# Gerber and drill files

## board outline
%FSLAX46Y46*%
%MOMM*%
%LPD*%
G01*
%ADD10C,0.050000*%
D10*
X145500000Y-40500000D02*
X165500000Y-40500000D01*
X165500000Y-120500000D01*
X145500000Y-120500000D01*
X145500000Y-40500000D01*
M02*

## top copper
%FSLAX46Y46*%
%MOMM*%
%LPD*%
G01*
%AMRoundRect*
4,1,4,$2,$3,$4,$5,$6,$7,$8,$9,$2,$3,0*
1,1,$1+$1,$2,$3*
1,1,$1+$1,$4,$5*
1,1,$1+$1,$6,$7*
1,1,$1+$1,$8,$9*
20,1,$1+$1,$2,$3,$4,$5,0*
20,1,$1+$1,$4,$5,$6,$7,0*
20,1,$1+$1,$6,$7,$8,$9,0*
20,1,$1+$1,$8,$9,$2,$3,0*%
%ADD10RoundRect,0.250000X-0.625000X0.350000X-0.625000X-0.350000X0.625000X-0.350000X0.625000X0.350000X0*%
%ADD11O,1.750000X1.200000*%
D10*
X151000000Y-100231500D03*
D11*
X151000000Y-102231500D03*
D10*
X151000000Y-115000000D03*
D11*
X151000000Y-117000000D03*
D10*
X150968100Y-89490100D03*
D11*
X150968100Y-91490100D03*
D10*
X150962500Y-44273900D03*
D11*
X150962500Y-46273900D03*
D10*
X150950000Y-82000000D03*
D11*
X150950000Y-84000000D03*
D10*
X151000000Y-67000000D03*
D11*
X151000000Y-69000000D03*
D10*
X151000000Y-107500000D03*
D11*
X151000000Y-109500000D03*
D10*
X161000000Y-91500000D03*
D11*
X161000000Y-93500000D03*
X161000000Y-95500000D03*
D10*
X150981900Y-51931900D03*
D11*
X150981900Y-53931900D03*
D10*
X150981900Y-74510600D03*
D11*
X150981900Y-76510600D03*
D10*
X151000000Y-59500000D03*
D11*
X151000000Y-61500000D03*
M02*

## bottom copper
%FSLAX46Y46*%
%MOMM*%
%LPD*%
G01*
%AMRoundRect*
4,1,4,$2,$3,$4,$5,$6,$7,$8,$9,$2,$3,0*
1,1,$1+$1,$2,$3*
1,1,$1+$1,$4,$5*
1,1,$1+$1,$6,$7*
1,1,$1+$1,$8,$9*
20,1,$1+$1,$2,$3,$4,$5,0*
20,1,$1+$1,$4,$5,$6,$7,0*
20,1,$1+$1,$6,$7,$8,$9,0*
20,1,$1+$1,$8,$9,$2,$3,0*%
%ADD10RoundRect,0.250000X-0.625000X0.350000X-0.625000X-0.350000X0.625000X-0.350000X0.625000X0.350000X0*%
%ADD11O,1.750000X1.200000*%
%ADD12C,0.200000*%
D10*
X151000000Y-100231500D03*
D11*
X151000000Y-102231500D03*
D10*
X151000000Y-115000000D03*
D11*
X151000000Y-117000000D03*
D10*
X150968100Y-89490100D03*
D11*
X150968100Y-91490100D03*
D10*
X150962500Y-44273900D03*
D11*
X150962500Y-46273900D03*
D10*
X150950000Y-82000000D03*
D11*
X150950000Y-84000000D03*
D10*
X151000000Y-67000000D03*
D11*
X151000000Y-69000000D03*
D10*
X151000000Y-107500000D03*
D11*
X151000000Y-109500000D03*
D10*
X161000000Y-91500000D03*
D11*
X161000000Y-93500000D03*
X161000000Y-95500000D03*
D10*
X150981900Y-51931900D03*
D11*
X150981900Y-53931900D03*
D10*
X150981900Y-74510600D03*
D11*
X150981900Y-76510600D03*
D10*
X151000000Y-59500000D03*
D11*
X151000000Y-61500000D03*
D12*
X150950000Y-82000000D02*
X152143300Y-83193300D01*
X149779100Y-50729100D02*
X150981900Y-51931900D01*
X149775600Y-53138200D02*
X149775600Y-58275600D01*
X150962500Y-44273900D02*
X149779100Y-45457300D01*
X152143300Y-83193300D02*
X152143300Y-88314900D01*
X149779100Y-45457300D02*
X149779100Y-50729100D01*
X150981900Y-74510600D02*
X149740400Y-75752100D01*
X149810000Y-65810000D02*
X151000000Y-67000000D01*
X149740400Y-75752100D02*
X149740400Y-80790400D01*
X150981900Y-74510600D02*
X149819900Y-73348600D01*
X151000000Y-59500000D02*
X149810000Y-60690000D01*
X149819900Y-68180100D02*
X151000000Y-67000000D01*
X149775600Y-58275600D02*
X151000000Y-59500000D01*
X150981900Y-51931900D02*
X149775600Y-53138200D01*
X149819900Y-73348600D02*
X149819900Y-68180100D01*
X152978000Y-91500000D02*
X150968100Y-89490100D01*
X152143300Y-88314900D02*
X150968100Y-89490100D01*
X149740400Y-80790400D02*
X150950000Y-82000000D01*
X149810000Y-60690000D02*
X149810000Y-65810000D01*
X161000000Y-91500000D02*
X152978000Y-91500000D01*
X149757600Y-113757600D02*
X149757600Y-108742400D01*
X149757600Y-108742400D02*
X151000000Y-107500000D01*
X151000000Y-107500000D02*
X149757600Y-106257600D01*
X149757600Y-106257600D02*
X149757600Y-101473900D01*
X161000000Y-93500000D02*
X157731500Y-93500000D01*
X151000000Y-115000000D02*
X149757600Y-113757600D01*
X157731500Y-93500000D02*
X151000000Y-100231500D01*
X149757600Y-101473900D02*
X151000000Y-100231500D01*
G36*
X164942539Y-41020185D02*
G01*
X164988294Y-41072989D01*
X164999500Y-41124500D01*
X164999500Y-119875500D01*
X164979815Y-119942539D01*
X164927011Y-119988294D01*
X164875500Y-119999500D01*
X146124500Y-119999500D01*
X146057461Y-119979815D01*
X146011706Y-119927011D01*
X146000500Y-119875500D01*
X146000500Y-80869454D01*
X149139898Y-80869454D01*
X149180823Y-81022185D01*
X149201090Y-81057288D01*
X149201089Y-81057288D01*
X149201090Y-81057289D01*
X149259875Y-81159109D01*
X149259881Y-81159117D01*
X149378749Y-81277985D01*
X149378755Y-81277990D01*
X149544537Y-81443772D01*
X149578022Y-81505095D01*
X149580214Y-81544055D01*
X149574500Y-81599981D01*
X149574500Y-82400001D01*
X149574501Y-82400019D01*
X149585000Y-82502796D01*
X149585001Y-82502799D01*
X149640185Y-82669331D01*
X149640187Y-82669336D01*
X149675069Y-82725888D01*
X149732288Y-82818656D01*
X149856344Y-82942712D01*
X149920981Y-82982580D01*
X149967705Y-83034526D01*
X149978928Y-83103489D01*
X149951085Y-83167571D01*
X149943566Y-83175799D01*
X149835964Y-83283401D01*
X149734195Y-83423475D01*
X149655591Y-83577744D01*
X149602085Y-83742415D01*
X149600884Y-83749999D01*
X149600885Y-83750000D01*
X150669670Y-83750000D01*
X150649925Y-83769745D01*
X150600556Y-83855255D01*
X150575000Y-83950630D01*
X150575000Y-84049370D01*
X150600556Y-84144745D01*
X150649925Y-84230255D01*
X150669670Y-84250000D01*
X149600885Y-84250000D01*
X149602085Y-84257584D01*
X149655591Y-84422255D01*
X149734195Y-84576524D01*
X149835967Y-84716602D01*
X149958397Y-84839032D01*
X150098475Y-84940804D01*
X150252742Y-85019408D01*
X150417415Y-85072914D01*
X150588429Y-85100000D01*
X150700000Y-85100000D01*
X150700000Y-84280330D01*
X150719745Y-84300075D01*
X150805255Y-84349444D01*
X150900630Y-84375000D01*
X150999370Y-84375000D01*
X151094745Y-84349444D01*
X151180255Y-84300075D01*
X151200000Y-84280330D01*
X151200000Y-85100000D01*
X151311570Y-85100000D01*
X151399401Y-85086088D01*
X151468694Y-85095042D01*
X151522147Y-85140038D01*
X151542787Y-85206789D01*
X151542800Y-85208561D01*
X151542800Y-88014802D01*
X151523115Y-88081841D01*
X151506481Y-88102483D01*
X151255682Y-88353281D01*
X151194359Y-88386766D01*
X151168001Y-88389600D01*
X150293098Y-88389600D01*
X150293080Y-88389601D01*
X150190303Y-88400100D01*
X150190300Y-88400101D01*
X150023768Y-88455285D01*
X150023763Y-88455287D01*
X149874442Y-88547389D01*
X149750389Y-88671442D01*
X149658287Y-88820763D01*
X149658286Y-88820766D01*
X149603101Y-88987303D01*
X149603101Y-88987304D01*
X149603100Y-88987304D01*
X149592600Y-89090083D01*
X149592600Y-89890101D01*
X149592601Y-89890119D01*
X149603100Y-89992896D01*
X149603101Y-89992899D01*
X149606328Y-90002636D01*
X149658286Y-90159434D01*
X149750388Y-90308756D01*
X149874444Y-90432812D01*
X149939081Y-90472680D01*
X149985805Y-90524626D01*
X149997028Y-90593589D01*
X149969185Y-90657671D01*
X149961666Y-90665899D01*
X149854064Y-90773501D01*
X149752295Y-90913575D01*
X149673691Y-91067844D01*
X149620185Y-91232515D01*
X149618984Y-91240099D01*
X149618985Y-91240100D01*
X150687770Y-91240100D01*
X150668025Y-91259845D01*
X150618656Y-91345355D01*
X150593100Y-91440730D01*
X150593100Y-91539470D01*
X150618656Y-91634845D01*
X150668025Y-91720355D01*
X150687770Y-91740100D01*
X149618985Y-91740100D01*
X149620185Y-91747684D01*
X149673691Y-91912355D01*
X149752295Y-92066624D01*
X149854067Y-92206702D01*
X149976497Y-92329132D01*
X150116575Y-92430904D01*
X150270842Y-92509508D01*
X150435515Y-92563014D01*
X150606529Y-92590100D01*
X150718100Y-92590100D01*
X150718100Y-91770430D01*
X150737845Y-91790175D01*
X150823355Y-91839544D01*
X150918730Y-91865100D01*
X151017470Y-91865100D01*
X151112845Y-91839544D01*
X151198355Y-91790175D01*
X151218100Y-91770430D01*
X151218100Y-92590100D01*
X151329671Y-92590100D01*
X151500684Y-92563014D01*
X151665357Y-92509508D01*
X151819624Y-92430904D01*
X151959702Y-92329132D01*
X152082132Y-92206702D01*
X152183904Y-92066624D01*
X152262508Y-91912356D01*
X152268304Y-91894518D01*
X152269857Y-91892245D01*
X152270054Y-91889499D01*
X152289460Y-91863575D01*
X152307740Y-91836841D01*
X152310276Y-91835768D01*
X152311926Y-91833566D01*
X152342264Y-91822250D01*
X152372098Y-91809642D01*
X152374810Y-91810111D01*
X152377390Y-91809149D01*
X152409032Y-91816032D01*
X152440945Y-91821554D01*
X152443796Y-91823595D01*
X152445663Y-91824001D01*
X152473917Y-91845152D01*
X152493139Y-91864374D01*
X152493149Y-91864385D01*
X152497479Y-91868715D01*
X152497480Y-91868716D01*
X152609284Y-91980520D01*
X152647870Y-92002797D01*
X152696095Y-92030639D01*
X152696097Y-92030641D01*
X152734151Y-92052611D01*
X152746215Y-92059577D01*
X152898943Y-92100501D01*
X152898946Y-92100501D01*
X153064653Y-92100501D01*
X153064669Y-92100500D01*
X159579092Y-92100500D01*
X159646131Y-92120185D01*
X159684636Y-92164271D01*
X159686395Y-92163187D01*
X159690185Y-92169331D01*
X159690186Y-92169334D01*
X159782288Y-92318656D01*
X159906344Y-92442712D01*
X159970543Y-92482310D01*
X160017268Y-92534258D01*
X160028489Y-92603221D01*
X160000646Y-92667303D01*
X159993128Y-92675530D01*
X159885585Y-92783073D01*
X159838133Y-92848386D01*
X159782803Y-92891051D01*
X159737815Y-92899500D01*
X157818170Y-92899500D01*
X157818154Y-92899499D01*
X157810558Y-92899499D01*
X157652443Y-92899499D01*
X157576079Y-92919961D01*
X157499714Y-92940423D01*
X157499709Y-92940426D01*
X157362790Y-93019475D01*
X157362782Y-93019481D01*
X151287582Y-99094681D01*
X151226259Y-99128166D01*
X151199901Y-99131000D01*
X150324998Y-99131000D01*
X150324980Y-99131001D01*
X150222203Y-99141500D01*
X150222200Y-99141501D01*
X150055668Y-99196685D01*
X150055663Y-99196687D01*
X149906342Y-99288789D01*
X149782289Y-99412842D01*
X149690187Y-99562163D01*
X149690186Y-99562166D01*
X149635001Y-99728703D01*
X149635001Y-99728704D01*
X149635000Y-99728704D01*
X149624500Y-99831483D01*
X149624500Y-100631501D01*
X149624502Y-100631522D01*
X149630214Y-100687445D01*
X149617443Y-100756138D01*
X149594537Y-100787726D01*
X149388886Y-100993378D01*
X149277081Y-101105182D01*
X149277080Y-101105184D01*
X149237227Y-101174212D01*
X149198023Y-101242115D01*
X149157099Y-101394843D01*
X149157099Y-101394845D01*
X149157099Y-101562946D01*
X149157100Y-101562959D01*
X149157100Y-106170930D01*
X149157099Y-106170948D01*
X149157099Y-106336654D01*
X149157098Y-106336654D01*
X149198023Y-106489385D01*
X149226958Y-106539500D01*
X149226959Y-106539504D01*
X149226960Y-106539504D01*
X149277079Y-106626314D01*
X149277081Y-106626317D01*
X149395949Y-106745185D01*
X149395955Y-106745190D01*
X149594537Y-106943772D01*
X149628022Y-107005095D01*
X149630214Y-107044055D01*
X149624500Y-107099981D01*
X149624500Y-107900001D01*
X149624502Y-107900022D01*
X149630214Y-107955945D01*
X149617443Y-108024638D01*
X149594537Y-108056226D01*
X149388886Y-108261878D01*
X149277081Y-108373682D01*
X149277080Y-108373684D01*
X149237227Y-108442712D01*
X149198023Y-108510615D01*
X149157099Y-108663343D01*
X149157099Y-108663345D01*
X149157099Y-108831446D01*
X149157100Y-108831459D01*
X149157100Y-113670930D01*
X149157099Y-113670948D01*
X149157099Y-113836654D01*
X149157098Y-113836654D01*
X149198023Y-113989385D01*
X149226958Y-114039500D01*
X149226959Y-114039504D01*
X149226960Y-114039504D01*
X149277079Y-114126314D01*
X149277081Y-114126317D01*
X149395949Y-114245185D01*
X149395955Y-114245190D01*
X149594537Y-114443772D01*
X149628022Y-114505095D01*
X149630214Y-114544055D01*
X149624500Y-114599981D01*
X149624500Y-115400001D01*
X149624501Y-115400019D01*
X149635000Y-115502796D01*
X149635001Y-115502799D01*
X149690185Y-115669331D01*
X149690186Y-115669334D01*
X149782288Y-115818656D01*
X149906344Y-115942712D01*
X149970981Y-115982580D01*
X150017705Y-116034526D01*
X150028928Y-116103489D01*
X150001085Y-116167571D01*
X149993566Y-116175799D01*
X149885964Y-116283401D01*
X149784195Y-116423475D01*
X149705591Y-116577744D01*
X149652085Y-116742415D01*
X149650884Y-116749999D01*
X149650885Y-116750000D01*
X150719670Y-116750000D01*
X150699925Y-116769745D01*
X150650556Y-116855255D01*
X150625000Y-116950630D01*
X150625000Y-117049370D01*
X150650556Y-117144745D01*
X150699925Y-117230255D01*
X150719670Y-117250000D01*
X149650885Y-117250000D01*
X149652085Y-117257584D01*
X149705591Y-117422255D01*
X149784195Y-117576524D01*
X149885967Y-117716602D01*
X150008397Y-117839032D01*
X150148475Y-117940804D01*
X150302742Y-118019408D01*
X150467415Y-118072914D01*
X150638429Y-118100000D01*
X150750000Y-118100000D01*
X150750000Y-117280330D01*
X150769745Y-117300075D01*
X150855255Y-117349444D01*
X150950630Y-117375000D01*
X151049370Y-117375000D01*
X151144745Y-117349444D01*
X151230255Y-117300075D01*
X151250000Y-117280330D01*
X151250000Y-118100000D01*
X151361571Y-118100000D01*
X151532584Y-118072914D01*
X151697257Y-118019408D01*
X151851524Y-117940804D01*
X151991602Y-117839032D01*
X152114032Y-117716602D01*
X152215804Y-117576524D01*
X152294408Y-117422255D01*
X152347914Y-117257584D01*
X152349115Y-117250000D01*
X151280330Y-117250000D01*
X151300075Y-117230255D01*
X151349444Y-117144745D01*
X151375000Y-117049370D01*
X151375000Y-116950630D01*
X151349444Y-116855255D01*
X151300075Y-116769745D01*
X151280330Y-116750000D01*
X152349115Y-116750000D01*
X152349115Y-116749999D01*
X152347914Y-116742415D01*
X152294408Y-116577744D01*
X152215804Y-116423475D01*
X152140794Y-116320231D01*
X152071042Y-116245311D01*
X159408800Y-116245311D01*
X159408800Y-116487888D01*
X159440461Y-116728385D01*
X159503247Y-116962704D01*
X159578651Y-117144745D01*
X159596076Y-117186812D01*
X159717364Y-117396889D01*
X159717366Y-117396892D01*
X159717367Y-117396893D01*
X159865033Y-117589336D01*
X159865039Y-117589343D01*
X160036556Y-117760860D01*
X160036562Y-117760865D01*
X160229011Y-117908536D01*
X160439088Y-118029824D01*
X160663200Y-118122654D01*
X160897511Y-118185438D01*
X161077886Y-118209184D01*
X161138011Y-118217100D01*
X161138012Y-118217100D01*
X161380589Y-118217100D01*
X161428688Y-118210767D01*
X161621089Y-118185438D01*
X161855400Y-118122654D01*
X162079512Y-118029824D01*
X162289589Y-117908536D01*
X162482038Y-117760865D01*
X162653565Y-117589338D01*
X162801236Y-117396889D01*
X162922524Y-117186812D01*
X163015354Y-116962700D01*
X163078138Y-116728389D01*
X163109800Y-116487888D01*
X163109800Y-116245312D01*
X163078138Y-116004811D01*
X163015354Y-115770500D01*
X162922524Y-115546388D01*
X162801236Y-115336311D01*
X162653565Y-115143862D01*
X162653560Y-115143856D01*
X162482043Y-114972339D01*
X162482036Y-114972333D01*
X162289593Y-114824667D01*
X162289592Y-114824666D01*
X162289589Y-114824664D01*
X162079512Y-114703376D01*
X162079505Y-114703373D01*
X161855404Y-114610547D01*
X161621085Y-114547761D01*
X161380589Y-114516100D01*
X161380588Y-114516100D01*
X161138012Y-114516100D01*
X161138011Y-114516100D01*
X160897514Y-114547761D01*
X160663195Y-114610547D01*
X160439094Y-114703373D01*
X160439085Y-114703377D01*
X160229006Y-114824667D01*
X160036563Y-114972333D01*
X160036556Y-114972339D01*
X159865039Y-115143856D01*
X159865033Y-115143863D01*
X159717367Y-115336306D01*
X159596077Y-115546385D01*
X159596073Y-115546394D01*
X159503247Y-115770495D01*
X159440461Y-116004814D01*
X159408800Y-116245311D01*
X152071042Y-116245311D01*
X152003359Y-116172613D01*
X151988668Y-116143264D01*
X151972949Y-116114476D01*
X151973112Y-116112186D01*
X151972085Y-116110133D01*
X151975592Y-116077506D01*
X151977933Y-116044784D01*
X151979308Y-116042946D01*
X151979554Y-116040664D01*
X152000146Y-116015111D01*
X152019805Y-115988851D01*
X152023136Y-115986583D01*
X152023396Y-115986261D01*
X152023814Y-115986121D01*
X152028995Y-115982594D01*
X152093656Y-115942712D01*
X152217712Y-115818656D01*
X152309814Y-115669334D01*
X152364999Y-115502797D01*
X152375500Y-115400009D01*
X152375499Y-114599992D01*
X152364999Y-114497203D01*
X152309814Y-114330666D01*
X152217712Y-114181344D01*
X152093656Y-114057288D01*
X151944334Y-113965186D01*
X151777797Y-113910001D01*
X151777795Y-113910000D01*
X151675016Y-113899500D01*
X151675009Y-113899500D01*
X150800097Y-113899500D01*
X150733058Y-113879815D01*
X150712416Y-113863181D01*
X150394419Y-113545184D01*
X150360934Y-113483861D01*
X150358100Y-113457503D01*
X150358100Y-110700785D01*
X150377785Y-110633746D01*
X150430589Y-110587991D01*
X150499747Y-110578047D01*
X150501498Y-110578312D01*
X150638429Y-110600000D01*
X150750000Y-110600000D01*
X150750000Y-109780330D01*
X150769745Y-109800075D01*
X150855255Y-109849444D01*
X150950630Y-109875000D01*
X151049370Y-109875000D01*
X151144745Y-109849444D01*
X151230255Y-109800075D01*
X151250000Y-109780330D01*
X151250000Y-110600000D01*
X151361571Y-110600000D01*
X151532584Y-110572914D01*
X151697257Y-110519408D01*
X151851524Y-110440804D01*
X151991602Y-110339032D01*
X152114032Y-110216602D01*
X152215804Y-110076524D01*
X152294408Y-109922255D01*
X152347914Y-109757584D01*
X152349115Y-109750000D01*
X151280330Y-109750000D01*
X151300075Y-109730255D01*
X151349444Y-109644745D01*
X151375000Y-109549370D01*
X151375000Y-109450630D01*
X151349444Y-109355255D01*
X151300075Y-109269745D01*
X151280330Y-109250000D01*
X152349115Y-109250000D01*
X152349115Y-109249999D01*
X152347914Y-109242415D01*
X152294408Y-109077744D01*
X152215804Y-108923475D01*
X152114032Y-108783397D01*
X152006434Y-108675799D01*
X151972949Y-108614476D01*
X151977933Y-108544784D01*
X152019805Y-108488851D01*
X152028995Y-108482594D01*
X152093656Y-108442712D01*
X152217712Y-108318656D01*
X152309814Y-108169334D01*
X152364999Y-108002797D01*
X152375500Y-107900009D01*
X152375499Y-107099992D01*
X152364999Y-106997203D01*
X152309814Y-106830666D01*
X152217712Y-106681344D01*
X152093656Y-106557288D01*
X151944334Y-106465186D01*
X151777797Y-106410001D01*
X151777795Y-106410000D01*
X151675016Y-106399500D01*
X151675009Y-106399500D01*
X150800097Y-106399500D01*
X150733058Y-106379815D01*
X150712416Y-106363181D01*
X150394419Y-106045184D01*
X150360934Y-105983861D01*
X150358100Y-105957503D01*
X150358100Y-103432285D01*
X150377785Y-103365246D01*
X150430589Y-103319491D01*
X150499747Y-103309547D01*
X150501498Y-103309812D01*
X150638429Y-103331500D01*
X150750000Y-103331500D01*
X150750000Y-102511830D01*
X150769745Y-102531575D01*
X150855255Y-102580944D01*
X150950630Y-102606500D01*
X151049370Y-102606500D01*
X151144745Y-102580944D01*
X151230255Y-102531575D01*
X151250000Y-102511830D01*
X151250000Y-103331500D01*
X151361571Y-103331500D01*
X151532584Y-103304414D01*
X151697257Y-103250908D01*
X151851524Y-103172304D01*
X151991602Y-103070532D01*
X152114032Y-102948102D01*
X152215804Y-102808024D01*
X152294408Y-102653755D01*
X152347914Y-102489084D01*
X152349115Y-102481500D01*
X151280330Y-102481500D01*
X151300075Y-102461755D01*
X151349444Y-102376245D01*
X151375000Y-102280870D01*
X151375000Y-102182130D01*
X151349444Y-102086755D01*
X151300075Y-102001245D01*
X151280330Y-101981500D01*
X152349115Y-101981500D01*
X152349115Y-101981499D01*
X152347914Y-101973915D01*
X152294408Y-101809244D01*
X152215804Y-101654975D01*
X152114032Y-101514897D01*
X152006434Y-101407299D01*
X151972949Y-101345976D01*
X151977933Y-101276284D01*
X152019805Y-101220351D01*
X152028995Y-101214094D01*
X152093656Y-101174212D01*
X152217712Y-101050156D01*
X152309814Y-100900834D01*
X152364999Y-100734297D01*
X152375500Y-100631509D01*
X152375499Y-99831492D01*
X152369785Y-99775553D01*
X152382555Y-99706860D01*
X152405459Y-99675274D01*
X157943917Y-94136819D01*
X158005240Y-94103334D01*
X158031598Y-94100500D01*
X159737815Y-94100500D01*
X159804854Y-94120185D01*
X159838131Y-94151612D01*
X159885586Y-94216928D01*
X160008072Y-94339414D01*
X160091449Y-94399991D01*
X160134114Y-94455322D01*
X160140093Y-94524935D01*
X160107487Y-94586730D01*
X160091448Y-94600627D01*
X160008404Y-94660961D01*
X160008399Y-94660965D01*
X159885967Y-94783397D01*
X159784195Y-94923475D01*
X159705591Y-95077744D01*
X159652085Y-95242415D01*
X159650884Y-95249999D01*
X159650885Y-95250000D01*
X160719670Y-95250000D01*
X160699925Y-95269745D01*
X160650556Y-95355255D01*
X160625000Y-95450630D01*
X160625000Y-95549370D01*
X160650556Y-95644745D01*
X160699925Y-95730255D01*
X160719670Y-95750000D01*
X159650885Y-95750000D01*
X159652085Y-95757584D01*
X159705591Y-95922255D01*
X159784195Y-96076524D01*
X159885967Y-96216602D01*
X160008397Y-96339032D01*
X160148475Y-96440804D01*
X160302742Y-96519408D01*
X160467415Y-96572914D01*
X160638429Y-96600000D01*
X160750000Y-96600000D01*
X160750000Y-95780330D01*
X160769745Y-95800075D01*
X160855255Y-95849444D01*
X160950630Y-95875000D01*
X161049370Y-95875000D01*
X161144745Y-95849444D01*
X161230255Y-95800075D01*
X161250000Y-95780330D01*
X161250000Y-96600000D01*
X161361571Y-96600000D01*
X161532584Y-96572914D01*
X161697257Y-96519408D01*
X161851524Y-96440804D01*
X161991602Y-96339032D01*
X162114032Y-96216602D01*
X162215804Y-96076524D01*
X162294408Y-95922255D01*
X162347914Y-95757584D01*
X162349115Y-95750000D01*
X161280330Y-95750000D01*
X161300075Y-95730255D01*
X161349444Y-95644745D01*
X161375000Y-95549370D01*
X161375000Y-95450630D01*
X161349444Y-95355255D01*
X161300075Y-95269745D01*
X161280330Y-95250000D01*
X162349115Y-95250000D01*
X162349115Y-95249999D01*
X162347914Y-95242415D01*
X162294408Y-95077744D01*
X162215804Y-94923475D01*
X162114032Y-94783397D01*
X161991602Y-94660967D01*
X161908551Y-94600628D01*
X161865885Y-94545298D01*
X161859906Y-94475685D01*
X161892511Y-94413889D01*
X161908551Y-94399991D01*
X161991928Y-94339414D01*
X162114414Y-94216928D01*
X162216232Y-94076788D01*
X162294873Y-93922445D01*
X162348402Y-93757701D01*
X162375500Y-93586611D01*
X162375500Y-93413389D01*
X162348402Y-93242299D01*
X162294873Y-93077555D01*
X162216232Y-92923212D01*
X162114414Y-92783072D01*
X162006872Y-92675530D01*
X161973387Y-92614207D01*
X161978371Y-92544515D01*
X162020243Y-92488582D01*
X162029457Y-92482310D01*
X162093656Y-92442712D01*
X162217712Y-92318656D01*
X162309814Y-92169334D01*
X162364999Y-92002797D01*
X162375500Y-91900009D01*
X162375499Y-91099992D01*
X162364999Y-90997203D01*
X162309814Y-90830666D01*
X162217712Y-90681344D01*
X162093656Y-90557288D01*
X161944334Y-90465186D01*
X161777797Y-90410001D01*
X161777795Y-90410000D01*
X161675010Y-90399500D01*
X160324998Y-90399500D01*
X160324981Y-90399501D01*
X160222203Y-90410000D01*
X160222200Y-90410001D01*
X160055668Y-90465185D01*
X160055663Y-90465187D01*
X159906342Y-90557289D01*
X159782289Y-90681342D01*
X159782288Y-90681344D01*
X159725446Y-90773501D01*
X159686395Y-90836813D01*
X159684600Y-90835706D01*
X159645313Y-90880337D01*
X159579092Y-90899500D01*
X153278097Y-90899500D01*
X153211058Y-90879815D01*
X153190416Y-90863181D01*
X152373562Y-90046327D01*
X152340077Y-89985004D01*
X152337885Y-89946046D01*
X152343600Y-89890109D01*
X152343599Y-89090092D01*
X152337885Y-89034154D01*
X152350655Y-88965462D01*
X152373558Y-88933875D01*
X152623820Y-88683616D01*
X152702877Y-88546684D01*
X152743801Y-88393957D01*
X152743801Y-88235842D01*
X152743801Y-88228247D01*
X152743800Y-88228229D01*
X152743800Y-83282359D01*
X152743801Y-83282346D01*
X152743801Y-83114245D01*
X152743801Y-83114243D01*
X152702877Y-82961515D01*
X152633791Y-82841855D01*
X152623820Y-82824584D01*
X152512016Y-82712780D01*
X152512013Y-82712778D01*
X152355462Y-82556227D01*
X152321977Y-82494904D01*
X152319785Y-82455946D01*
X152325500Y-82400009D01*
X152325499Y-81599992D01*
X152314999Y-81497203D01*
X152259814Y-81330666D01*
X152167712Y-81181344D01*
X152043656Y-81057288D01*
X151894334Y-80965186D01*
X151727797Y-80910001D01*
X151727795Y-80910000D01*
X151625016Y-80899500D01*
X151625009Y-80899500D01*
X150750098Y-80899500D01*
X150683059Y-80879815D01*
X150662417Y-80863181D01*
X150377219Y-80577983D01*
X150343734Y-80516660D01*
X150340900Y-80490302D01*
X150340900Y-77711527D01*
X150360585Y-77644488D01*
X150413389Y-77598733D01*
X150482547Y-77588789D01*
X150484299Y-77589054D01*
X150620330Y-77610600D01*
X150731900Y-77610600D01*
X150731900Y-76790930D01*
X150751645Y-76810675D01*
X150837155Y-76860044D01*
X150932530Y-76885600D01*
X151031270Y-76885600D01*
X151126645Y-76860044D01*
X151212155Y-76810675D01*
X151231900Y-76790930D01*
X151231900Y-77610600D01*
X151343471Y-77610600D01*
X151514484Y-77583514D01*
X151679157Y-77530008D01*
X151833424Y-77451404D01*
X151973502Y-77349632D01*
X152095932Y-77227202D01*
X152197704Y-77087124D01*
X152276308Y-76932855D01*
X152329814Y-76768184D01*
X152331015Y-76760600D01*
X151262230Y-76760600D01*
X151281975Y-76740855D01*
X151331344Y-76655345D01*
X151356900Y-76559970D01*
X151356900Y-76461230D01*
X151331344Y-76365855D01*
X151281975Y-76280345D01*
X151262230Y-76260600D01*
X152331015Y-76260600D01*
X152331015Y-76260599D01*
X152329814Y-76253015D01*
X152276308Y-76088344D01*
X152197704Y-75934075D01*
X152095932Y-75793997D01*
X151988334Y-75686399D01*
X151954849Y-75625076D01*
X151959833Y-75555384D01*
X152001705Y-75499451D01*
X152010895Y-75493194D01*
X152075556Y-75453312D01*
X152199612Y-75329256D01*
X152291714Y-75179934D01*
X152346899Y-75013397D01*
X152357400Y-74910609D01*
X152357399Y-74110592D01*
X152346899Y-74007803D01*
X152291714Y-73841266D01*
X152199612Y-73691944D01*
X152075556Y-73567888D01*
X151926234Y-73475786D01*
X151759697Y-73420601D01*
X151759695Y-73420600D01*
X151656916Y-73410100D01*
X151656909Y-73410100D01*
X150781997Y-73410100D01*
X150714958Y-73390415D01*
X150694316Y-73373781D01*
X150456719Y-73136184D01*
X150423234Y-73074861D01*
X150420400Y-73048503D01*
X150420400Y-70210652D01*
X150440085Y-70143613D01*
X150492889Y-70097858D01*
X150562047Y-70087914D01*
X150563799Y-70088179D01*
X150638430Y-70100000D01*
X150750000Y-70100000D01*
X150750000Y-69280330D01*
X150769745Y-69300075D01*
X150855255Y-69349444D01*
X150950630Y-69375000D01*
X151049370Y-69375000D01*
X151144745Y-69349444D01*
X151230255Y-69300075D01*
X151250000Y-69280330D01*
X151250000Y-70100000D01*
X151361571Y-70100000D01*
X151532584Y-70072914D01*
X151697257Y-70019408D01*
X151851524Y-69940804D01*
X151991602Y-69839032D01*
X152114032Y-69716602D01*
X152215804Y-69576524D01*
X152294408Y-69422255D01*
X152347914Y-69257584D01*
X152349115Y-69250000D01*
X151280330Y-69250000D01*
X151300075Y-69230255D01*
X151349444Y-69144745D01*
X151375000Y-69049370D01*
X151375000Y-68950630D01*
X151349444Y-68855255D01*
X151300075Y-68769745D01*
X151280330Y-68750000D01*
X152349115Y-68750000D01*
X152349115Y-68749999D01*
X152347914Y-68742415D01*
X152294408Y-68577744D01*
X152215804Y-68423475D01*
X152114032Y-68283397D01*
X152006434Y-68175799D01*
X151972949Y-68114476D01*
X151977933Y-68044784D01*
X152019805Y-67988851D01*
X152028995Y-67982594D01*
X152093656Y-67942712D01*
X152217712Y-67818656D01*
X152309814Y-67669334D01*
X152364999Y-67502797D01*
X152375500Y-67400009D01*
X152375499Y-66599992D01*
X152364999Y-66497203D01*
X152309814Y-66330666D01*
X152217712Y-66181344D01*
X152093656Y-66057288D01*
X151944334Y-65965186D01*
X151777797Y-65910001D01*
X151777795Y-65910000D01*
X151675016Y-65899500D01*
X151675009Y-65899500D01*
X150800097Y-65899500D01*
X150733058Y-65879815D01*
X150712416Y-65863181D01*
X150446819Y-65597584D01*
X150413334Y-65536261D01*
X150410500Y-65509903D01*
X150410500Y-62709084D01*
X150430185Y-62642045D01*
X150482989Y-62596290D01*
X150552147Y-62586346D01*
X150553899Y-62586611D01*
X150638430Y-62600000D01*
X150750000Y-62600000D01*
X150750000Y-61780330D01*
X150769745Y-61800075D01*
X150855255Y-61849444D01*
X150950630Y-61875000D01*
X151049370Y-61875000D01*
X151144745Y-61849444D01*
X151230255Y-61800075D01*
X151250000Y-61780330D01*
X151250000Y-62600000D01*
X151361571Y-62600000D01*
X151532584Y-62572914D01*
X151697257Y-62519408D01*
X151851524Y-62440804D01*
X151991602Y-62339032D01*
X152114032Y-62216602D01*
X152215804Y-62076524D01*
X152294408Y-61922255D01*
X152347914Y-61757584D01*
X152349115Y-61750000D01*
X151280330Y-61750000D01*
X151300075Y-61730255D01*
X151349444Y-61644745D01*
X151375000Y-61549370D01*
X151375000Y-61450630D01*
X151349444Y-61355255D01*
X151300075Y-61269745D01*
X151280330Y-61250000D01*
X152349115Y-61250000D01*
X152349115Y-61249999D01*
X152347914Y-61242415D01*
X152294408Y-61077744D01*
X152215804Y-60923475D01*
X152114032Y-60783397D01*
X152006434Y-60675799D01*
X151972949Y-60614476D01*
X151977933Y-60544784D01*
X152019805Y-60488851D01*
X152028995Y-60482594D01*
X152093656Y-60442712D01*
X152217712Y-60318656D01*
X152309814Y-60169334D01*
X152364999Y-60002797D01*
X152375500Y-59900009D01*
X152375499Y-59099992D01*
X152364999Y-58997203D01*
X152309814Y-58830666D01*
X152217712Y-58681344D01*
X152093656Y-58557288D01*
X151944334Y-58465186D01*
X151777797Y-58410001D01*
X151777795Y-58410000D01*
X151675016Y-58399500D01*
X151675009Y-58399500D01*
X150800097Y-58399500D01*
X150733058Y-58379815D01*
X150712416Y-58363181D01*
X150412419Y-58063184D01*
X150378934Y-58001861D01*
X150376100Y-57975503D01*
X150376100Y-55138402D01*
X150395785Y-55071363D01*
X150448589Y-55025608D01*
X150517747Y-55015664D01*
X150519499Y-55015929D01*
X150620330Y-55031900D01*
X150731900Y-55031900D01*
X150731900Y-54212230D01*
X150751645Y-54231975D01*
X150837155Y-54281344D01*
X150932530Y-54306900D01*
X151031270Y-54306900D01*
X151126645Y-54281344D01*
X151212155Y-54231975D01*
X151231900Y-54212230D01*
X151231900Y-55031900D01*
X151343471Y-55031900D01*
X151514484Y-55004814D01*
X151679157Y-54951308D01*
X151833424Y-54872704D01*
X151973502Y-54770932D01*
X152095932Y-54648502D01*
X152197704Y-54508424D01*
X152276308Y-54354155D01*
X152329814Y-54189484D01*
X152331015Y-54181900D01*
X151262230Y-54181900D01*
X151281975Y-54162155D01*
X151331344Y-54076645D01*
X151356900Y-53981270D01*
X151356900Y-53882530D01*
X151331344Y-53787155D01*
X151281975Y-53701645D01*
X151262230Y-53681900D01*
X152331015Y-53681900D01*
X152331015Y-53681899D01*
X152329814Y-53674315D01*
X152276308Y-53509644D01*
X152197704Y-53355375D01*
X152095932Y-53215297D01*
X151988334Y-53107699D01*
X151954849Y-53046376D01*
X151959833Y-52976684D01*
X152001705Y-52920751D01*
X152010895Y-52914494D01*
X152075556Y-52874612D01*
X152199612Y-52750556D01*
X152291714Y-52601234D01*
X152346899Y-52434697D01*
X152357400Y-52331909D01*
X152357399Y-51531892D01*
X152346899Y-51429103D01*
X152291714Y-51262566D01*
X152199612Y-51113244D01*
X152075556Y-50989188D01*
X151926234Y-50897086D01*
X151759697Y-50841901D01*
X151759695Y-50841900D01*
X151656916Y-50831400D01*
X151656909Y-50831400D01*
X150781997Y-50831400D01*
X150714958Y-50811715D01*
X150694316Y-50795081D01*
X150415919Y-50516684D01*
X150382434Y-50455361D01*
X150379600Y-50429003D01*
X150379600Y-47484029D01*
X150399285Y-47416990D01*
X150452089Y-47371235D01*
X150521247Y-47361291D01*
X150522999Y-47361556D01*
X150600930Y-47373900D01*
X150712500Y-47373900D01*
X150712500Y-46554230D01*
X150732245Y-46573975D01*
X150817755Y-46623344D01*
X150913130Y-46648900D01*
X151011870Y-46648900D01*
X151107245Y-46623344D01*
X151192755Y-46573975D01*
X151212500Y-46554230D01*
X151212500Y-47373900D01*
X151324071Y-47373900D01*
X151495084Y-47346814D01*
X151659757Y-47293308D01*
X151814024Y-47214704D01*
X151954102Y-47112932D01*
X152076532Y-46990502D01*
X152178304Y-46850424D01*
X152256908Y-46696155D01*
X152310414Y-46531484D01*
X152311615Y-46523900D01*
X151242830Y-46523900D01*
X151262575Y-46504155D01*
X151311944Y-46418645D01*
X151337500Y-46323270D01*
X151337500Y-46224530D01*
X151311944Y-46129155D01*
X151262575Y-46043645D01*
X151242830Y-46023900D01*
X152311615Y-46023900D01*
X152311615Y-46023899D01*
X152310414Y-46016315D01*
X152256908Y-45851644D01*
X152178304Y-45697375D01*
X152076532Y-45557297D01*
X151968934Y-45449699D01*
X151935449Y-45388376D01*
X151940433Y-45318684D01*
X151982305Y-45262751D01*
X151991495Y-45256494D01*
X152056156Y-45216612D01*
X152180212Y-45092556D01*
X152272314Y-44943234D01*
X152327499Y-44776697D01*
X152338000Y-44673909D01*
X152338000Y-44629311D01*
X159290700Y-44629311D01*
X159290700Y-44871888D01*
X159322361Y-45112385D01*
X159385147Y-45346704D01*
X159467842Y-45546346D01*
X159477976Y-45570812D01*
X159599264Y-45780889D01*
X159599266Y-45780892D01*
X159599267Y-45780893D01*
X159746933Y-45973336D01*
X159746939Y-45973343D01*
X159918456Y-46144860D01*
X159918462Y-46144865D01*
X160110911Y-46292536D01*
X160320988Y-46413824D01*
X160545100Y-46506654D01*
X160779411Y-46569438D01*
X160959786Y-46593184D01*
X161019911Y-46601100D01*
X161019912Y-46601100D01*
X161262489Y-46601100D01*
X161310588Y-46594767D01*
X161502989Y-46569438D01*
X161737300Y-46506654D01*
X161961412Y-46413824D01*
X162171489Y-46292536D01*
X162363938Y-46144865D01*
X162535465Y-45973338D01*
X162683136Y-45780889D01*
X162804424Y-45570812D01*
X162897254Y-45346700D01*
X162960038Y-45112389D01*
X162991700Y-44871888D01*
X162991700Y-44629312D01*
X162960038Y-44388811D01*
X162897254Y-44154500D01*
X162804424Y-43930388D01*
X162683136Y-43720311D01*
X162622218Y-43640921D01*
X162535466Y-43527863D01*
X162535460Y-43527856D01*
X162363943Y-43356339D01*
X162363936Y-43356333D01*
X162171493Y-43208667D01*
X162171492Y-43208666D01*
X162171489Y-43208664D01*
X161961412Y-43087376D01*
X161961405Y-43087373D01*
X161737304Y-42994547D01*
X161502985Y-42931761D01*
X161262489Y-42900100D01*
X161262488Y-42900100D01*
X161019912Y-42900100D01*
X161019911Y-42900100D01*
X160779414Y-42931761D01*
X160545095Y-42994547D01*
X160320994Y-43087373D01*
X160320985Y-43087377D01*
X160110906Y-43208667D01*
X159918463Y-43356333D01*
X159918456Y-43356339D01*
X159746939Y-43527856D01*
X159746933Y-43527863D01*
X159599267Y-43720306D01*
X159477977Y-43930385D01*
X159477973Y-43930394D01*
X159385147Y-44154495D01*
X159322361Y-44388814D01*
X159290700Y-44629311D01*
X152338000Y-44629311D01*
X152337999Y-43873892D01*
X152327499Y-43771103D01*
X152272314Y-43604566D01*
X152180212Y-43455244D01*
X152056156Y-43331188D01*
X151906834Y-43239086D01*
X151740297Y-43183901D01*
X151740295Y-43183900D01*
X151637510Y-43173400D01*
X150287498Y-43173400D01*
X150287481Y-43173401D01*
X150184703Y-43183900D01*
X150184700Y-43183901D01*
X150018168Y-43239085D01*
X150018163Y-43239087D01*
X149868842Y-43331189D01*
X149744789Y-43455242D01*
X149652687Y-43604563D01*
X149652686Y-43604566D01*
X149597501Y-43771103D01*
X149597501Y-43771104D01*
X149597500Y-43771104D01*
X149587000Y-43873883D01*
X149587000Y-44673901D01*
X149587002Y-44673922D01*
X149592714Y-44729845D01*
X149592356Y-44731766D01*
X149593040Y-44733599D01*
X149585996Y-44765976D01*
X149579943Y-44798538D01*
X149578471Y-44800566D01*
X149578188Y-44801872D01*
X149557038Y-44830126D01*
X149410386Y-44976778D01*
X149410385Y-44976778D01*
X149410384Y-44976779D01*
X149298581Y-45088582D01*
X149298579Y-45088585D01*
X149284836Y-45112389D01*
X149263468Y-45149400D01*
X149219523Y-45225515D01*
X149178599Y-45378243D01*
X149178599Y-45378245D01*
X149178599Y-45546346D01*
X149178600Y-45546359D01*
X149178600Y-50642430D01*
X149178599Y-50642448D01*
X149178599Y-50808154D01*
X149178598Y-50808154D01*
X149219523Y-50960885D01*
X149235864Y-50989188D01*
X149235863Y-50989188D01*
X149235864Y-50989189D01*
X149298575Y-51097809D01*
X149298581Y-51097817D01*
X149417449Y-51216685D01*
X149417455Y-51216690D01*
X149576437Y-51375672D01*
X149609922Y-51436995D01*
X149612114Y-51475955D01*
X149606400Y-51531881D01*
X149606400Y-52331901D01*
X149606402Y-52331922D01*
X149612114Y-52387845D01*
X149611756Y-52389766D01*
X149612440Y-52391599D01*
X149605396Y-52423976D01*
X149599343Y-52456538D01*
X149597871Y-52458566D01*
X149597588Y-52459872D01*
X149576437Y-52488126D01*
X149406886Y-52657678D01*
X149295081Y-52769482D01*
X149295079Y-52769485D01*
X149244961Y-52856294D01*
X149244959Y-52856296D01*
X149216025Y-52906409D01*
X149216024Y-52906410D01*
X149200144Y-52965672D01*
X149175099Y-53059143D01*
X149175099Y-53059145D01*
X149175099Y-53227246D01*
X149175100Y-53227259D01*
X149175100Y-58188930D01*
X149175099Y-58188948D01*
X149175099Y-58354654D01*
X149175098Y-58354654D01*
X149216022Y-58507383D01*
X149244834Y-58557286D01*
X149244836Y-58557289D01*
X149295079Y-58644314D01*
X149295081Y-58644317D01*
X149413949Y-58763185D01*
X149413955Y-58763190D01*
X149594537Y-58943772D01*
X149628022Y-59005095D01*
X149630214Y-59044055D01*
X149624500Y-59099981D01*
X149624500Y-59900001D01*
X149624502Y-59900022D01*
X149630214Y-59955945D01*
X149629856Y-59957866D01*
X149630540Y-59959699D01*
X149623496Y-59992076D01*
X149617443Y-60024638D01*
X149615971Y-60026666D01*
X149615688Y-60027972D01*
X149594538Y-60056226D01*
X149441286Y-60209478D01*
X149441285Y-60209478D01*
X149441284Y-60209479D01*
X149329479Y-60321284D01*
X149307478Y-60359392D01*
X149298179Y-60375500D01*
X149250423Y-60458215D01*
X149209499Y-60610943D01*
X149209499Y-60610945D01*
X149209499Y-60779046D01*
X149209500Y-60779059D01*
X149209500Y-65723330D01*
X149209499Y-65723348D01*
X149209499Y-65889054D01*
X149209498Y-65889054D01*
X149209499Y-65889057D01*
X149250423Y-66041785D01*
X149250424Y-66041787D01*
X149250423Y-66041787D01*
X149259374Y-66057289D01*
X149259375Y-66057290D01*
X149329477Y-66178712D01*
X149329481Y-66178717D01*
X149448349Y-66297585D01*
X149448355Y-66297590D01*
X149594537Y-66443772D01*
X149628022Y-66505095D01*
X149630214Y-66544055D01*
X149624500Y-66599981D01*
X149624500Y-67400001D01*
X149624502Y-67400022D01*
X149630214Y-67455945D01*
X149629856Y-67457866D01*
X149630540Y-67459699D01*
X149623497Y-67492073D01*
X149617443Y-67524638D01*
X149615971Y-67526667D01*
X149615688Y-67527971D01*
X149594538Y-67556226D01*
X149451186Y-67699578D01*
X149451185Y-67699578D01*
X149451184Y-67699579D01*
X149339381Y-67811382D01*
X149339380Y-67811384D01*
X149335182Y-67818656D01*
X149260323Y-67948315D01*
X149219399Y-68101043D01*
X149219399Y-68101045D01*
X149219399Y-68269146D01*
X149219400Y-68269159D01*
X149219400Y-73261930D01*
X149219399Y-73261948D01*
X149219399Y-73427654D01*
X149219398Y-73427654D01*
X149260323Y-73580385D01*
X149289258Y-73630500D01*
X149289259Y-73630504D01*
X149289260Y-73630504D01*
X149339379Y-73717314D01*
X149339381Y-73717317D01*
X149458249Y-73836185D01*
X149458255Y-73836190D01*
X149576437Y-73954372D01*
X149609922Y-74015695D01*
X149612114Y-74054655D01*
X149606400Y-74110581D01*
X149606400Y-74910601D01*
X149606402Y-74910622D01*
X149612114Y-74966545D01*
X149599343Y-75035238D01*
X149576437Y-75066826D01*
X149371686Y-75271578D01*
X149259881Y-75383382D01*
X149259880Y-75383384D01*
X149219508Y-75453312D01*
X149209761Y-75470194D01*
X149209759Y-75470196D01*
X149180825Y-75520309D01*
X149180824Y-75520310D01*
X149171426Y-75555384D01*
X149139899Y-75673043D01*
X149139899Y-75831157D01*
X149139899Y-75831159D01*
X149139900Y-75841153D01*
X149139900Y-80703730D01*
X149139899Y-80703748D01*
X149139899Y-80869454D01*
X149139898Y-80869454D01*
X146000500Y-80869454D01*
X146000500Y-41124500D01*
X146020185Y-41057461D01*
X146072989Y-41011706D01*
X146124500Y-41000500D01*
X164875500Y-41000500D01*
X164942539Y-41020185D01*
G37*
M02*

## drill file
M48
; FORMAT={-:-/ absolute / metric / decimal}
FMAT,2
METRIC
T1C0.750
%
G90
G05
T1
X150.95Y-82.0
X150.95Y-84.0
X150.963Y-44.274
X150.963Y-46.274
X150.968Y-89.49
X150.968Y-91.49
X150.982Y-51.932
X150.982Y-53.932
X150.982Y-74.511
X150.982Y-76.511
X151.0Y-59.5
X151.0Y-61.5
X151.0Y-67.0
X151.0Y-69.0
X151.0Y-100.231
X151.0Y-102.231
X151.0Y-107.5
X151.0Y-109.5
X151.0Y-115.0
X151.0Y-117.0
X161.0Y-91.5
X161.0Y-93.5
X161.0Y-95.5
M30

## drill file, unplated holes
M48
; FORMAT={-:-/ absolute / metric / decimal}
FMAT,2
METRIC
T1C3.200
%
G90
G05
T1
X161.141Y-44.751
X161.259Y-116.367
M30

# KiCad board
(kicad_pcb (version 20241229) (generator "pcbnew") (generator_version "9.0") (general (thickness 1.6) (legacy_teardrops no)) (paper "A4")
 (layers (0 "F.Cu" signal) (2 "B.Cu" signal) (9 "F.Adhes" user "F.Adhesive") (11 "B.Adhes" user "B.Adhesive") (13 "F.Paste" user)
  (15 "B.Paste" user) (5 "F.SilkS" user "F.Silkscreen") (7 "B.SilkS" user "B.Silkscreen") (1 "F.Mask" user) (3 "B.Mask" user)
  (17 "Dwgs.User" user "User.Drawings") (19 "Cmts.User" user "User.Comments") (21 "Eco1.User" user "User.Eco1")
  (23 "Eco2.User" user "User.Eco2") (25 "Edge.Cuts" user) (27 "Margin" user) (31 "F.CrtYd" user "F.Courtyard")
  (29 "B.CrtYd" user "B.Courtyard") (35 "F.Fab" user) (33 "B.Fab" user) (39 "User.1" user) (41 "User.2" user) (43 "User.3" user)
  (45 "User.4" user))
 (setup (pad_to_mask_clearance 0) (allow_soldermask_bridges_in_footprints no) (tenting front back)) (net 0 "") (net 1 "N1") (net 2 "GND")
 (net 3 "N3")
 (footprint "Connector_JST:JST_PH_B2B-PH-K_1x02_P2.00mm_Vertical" (layer "F.Cu") (at 151 100.2315 -90)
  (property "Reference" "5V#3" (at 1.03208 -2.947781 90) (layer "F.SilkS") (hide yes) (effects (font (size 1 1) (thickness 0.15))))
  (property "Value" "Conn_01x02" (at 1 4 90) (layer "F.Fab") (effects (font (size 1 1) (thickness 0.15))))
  (pad "1" thru_hole roundrect (at 0 0 270) (size 1.2 1.75) (drill 0.75) (layers "*.Cu" "*.Mask") (remove_unused_layers no)
   (roundrect_rratio 0.208333) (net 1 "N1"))
  (pad "2" thru_hole oval (at 2 0 270) (size 1.2 1.75) (drill 0.75) (layers "*.Cu" "*.Mask") (remove_unused_layers no) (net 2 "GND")))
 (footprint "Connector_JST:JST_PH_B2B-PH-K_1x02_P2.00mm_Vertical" (layer "F.Cu") (at 151 115 -90)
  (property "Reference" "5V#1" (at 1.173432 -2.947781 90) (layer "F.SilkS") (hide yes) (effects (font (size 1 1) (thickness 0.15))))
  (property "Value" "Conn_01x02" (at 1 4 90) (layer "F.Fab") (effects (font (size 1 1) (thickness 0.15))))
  (pad "1" thru_hole roundrect (at 0 0 270) (size 1.2 1.75) (drill 0.75) (layers "*.Cu" "*.Mask") (remove_unused_layers no)
   (roundrect_rratio 0.208333) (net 1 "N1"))
  (pad "2" thru_hole oval (at 2 0 270) (size 1.2 1.75) (drill 0.75) (layers "*.Cu" "*.Mask") (remove_unused_layers no) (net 2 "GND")))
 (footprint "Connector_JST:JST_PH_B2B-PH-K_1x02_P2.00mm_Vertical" (layer "F.Cu") (at 150.9681 89.4901 -90)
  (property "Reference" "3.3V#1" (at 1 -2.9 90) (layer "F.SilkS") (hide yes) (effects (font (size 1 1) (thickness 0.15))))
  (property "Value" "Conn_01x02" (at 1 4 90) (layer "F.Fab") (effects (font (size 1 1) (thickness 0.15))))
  (pad "1" thru_hole roundrect (at 0 0 270) (size 1.2 1.75) (drill 0.75) (layers "*.Cu" "*.Mask") (remove_unused_layers no)
   (roundrect_rratio 0.208333) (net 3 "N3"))
  (pad "2" thru_hole oval (at 2 0 270) (size 1.2 1.75) (drill 0.75) (layers "*.Cu" "*.Mask") (remove_unused_layers no) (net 2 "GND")))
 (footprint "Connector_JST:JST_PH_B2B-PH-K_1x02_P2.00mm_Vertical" (layer "F.Cu") (at 150.9625 44.2739 -90)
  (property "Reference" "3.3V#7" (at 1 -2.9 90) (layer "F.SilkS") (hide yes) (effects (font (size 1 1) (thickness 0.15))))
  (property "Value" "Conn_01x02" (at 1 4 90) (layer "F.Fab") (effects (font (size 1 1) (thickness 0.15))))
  (pad "1" thru_hole roundrect (at 0 0 270) (size 1.2 1.75) (drill 0.75) (layers "*.Cu" "*.Mask") (remove_unused_layers no)
   (roundrect_rratio 0.208333) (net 3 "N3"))
  (pad "2" thru_hole oval (at 2 0 270) (size 1.2 1.75) (drill 0.75) (layers "*.Cu" "*.Mask") (remove_unused_layers no) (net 2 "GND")))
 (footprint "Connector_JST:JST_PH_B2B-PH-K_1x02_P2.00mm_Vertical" (layer "F.Cu") (at 150.95 82 -90)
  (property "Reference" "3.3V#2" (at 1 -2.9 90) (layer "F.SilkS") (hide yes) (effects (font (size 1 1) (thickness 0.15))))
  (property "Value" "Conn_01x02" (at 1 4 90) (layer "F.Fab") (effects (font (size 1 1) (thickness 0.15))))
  (pad "1" thru_hole roundrect (at 0 0 270) (size 1.2 1.75) (drill 0.75) (layers "*.Cu" "*.Mask") (remove_unused_layers no)
   (roundrect_rratio 0.208333) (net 3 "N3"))
  (pad "2" thru_hole oval (at 2 0 270) (size 1.2 1.75) (drill 0.75) (layers "*.Cu" "*.Mask") (remove_unused_layers no) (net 2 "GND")))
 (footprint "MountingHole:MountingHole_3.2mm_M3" (layer "F.Cu") (at 161.2593 116.3666)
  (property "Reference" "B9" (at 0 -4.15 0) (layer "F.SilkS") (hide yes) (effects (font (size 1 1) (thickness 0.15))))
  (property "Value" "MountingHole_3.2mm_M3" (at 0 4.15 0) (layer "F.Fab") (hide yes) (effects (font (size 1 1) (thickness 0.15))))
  (pad "" np_thru_hole circle (at 0 0) (size 3.2 3.2) (drill 3.2) (layers "*.Cu" "*.Mask")))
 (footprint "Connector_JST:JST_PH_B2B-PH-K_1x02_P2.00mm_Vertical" (layer "F.Cu") (at 151 67 -90)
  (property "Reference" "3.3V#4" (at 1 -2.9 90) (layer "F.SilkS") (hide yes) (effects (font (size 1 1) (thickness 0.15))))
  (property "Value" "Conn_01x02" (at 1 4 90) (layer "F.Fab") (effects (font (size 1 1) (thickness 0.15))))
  (pad "1" thru_hole roundrect (at 0 0 270) (size 1.2 1.75) (drill 0.75) (layers "*.Cu" "*.Mask") (remove_unused_layers no)
   (roundrect_rratio 0.208333) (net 3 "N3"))
  (pad "2" thru_hole oval (at 2 0 270) (size 1.2 1.75) (drill 0.75) (layers "*.Cu" "*.Mask") (remove_unused_layers no) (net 2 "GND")))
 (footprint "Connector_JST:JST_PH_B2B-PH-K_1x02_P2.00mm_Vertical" (layer "F.Cu") (at 151 107.5 -90)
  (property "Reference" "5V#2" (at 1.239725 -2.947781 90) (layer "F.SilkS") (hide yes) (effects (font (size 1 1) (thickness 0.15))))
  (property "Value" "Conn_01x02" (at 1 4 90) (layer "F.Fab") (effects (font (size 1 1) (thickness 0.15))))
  (pad "1" thru_hole roundrect (at 0 0 270) (size 1.2 1.75) (drill 0.75) (layers "*.Cu" "*.Mask") (remove_unused_layers no)
   (roundrect_rratio 0.208333) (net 1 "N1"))
  (pad "2" thru_hole oval (at 2 0 270) (size 1.2 1.75) (drill 0.75) (layers "*.Cu" "*.Mask") (remove_unused_layers no) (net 2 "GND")))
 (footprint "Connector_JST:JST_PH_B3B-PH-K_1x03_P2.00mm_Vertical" (layer "F.Cu") (at 161 91.5 -90)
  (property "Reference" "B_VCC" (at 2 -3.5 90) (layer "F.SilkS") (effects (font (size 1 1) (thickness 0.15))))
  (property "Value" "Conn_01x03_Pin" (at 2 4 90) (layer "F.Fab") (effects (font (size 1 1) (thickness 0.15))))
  (pad "1" thru_hole roundrect (at 0 0 270) (size 1.2 1.75) (drill 0.75) (layers "*.Cu" "*.Mask") (remove_unused_layers no)
   (roundrect_rratio 0.208333) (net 3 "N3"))
  (pad "2" thru_hole oval (at 2 0 270) (size 1.2 1.75) (drill 0.75) (layers "*.Cu" "*.Mask") (remove_unused_layers no) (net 1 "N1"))
  (pad "3" thru_hole oval (at 4 0 270) (size 1.2 1.75) (drill 0.75) (layers "*.Cu" "*.Mask") (remove_unused_layers no) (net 2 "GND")))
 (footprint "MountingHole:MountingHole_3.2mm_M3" (layer "F.Cu") (at 161.1412 44.7506)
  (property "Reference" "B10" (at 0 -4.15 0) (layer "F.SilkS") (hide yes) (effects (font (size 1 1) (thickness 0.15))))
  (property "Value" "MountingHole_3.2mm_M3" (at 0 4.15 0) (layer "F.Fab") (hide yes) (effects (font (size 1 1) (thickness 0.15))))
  (pad "" np_thru_hole circle (at 0 0) (size 3.2 3.2) (drill 3.2) (layers "*.Cu" "*.Mask")))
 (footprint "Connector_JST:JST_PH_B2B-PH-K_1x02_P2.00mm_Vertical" (layer "F.Cu") (at 150.9819 51.9319 -90)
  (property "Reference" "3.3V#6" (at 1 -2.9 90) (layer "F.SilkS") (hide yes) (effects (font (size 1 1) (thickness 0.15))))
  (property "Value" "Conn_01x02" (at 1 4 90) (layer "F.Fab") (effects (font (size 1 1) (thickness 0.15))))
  (pad "1" thru_hole roundrect (at 0 0 270) (size 1.2 1.75) (drill 0.75) (layers "*.Cu" "*.Mask") (remove_unused_layers no)
   (roundrect_rratio 0.208333) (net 3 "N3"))
  (pad "2" thru_hole oval (at 2 0 270) (size 1.2 1.75) (drill 0.75) (layers "*.Cu" "*.Mask") (remove_unused_layers no) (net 2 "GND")))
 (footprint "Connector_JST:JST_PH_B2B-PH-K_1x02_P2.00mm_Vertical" (layer "F.Cu") (at 150.9819 74.5106 -90)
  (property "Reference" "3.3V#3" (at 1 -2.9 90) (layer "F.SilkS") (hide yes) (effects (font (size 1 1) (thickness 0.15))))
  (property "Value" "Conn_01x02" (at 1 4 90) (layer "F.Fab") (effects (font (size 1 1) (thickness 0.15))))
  (pad "1" thru_hole roundrect (at 0 0 270) (size 1.2 1.75) (drill 0.75) (layers "*.Cu" "*.Mask") (remove_unused_layers no)
   (roundrect_rratio 0.208333) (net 3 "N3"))
  (pad "2" thru_hole oval (at 2 0 270) (size 1.2 1.75) (drill 0.75) (layers "*.Cu" "*.Mask") (remove_unused_layers no) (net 2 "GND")))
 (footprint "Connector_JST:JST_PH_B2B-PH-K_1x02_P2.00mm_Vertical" (layer "F.Cu") (at 151 59.5 -90)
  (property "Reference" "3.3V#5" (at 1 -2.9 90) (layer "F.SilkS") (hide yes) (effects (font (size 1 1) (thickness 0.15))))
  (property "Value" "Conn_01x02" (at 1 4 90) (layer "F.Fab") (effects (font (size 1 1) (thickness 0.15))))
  (pad "1" thru_hole roundrect (at 0 0 270) (size 1.2 1.75) (drill 0.75) (layers "*.Cu" "*.Mask") (remove_unused_layers no)
   (roundrect_rratio 0.208333) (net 3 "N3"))
  (pad "2" thru_hole oval (at 2 0 270) (size 1.2 1.75) (drill 0.75) (layers "*.Cu" "*.Mask") (remove_unused_layers no) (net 2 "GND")))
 (gr_rect (start 145.5 40.5) (end 165.5 120.5) (stroke (width 0.05) (type default)) (fill no) (layer "Edge.Cuts"))
 (segment (start 150.95 82) (end 152.1433 83.1933) (width 0.2) (layer "B.Cu") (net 3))
 (segment (start 149.7791 50.7291) (end 150.9819 51.9319) (width 0.2) (layer "B.Cu") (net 3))
 (segment (start 149.7756 53.1382) (end 149.7756 58.2756) (width 0.2) (layer "B.Cu") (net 3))
 (segment (start 150.9625 44.2739) (end 149.7791 45.4573) (width 0.2) (layer "B.Cu") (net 3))
 (segment (start 152.1433 83.1933) (end 152.1433 88.3149) (width 0.2) (layer "B.Cu") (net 3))
 (segment (start 149.7791 45.4573) (end 149.7791 50.7291) (width 0.2) (layer "B.Cu") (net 3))
 (segment (start 150.9819 74.5106) (end 149.7404 75.7521) (width 0.2) (layer "B.Cu") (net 3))
 (segment (start 149.81 65.81) (end 151 67) (width 0.2) (layer "B.Cu") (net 3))
 (segment (start 149.7404 75.7521) (end 149.7404 80.7904) (width 0.2) (layer "B.Cu") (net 3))
 (segment (start 150.9819 74.5106) (end 149.8199 73.3486) (width 0.2) (layer "B.Cu") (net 3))
 (segment (start 151 59.5) (end 149.81 60.69) (width 0.2) (layer "B.Cu") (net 3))
 (segment (start 149.8199 68.1801) (end 151 67) (width 0.2) (layer "B.Cu") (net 3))
 (segment (start 149.7756 58.2756) (end 151 59.5) (width 0.2) (layer "B.Cu") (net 3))
 (segment (start 150.9819 51.9319) (end 149.7756 53.1382) (width 0.2) (layer "B.Cu") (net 3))
 (segment (start 149.8199 73.3486) (end 149.8199 68.1801) (width 0.2) (layer "B.Cu") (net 3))
 (segment (start 152.978 91.5) (end 150.9681 89.4901) (width 0.2) (layer "B.Cu") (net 3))
 (segment (start 152.1433 88.3149) (end 150.9681 89.4901) (width 0.2) (layer "B.Cu") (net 3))
 (segment (start 149.7404 80.7904) (end 150.95 82) (width 0.2) (layer "B.Cu") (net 3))
 (segment (start 149.81 60.69) (end 149.81 65.81) (width 0.2) (layer "B.Cu") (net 3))
 (segment (start 161 91.5) (end 152.978 91.5) (width 0.2) (layer "B.Cu") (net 3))
 (segment (start 149.7576 113.7576) (end 149.7576 108.7424) (width 0.2) (layer "B.Cu") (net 1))
 (segment (start 149.7576 108.7424) (end 151 107.5) (width 0.2) (layer "B.Cu") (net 1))
 (segment (start 151 107.5) (end 149.7576 106.2576) (width 0.2) (layer "B.Cu") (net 1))
 (segment (start 149.7576 106.2576) (end 149.7576 101.4739) (width 0.2) (layer "B.Cu") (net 1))
 (segment (start 161 93.5) (end 157.7315 93.5) (width 0.2) (layer "B.Cu") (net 1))
 (segment (start 151 115) (end 149.7576 113.7576) (width 0.2) (layer "B.Cu") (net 1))
 (segment (start 157.7315 93.5) (end 151 100.2315) (width 0.2) (layer "B.Cu") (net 1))
 (segment (start 149.7576 101.4739) (end 151 100.2315) (width 0.2) (layer "B.Cu") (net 1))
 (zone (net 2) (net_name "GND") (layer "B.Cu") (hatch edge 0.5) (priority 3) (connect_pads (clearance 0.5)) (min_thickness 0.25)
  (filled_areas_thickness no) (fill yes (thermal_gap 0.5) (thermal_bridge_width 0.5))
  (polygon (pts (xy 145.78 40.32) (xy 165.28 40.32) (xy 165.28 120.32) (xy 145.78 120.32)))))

